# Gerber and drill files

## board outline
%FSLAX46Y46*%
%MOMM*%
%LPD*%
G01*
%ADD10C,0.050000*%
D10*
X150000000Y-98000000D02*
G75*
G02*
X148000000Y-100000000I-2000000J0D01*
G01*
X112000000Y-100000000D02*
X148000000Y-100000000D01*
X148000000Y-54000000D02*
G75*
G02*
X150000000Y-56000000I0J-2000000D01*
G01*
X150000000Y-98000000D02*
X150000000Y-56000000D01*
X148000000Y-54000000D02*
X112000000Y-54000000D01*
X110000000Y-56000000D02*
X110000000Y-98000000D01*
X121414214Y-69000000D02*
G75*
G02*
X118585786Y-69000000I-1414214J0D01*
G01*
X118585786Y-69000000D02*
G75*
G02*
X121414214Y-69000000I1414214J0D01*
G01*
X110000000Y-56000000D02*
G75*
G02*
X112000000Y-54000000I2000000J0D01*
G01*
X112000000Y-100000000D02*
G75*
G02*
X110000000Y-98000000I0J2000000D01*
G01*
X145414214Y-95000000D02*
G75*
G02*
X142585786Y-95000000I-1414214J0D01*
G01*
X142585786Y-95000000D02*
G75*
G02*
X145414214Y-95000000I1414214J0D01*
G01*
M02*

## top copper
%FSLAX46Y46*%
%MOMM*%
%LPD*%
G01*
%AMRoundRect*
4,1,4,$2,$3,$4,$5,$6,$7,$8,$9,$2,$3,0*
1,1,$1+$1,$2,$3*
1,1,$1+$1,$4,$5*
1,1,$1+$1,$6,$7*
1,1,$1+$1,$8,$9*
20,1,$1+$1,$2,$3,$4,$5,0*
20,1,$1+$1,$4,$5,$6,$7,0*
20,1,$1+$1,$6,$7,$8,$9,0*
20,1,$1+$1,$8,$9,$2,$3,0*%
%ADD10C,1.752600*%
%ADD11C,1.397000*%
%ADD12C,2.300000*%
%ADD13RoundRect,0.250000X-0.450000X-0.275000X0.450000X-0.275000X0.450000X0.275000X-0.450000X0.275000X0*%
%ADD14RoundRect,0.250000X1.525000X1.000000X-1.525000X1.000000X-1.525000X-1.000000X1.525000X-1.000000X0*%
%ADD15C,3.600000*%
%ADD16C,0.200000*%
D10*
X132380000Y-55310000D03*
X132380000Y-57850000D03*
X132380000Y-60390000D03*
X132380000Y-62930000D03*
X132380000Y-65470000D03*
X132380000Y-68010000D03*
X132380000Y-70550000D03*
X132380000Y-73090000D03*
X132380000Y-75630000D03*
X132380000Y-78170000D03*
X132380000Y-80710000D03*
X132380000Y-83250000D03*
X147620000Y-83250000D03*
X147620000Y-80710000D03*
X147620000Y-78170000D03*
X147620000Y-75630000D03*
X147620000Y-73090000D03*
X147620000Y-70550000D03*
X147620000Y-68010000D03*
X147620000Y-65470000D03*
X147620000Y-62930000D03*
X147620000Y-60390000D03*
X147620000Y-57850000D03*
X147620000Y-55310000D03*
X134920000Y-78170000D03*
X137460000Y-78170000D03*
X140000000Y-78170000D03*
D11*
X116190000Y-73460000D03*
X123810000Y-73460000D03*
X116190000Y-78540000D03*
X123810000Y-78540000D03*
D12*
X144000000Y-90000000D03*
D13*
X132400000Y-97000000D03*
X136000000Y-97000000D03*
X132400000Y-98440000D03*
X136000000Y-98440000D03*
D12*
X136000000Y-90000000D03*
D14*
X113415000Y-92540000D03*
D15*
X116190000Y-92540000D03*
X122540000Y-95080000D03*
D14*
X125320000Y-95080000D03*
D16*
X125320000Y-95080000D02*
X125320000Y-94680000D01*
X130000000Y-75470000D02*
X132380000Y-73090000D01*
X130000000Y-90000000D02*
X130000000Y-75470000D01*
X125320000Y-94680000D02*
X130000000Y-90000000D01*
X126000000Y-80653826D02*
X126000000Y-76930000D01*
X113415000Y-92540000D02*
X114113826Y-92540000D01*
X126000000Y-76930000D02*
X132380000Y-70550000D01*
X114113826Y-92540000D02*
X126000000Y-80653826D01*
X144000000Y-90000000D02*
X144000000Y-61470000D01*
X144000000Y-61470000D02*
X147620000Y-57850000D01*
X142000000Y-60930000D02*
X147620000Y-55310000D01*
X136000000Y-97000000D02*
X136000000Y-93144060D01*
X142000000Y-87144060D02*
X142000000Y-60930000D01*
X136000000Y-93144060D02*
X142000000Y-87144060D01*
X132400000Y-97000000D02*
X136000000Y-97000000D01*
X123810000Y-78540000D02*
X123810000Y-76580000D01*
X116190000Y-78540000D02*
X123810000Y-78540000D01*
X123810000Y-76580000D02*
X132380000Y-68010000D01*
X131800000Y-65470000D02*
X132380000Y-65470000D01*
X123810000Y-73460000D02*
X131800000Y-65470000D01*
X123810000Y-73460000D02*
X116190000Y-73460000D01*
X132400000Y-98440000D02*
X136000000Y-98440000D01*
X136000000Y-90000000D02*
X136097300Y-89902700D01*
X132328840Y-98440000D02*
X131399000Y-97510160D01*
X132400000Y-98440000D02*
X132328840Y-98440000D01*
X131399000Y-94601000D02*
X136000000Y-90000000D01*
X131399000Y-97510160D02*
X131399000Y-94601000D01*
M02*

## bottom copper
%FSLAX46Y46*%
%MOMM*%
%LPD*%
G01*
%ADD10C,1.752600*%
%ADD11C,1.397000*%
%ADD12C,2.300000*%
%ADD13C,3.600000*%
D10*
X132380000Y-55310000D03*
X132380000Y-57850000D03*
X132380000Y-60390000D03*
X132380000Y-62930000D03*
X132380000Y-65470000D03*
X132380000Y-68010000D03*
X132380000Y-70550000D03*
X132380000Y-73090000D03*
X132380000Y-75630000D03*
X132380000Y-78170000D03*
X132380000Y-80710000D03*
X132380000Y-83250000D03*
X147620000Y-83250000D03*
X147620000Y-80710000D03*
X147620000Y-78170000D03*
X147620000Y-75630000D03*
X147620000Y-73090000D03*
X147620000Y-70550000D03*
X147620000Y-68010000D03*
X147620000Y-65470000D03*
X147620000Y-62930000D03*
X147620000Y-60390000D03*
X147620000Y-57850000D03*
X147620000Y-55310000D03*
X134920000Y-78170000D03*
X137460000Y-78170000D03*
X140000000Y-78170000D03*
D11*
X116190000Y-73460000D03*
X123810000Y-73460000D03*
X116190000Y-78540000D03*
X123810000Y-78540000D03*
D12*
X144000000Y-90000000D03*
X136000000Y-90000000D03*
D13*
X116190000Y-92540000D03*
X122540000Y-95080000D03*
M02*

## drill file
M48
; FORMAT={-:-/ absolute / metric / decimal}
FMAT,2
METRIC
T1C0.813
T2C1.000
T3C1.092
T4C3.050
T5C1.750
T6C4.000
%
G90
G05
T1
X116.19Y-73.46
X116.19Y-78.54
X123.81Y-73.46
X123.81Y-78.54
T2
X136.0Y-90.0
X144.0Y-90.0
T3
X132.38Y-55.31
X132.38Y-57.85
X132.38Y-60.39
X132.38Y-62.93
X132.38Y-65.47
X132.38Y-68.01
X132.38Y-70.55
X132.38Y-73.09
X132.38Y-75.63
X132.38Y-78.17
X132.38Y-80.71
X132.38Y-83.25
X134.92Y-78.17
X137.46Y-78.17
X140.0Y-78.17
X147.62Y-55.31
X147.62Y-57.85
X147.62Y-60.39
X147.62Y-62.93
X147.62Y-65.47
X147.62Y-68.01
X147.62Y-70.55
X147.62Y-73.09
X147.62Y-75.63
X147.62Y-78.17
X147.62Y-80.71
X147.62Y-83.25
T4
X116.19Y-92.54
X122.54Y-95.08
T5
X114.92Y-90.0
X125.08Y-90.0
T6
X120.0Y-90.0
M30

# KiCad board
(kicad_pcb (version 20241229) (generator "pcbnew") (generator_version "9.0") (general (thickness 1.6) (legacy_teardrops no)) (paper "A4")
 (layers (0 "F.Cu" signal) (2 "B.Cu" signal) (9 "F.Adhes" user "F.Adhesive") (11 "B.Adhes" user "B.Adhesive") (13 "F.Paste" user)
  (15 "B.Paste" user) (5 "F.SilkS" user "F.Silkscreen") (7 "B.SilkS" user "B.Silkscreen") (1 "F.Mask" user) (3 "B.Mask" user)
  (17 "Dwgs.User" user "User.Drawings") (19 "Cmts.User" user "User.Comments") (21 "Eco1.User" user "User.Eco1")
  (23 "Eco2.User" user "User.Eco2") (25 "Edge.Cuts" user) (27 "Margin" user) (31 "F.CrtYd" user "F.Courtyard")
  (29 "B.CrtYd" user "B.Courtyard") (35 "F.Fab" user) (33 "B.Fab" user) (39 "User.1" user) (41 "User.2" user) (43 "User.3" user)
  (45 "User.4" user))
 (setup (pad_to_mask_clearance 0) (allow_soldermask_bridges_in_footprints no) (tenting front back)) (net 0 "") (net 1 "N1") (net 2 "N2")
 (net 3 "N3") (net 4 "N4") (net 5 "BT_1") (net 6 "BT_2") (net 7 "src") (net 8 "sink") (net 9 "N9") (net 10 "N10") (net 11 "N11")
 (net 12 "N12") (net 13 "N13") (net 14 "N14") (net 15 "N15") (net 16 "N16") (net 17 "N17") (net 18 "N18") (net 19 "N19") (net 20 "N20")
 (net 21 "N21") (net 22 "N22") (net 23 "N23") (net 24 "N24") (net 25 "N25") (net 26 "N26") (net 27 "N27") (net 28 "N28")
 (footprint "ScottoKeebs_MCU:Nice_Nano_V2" (layer "F.Cu") (at 140 69)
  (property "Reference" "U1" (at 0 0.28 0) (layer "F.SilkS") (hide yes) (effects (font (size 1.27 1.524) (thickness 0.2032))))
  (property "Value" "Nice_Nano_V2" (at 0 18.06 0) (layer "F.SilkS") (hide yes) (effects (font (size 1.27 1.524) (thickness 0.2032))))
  (pad "1" thru_hole circle (at -7.62 -13.69 270) (size 1.7526 1.7526) (drill 1.0922) (layers "*.Cu" "*.Mask") (remove_unused_layers no)
   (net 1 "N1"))
  (pad "2" thru_hole circle (at -7.62 -11.15 270) (size 1.7526 1.7526) (drill 1.0922) (layers "*.Cu" "*.Mask") (remove_unused_layers no)
   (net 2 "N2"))
  (pad "3" thru_hole circle (at -7.62 -8.61 270) (size 1.7526 1.7526) (drill 1.0922) (layers "*.Cu" "*.Mask") (remove_unused_layers no)
   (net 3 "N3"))
  (pad "4" thru_hole circle (at -7.62 -6.07 270) (size 1.7526 1.7526) (drill 1.0922) (layers "*.Cu" "*.Mask") (remove_unused_layers no)
   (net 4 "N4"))
  (pad "5" thru_hole circle (at -7.62 -3.53 270) (size 1.7526 1.7526) (drill 1.0922) (layers "*.Cu" "*.Mask") (remove_unused_layers no)
   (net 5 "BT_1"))
  (pad "6" thru_hole circle (at -7.62 -0.99 270) (size 1.7526 1.7526) (drill 1.0922) (layers "*.Cu" "*.Mask") (remove_unused_layers no)
   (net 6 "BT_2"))
  (pad "7" thru_hole circle (at -7.62 1.55 270) (size 1.7526 1.7526) (drill 1.0922) (layers "*.Cu" "*.Mask") (remove_unused_layers no)
   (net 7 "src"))
  (pad "8" thru_hole circle (at -7.62 4.09 270) (size 1.7526 1.7526) (drill 1.0922) (layers "*.Cu" "*.Mask") (remove_unused_layers no)
   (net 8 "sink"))
  (pad "9" thru_hole circle (at -7.62 6.63 270) (size 1.7526 1.7526) (drill 1.0922) (layers "*.Cu" "*.Mask") (remove_unused_layers no)
   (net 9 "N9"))
  (pad "10" thru_hole circle (at -7.62 9.17 270) (size 1.7526 1.7526) (drill 1.0922) (layers "*.Cu" "*.Mask") (remove_unused_layers no)
   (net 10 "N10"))
  (pad "11" thru_hole circle (at -7.62 11.71 270) (size 1.7526 1.7526) (drill 1.0922) (layers "*.Cu" "*.Mask") (remove_unused_layers no)
   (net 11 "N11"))
  (pad "12" thru_hole circle (at -7.62 14.25 270) (size 1.7526 1.7526) (drill 1.0922) (layers "*.Cu" "*.Mask") (remove_unused_layers no)
   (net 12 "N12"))
  (pad "13" thru_hole circle (at 7.62 14.25 270) (size 1.7526 1.7526) (drill 1.0922) (layers "*.Cu" "*.Mask") (remove_unused_layers no)
   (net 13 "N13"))
  (pad "14" thru_hole circle (at 7.62 11.71 270) (size 1.7526 1.7526) (drill 1.0922) (layers "*.Cu" "*.Mask") (remove_unused_layers no)
   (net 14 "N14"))
  (pad "15" thru_hole circle (at 7.62 9.17 270) (size 1.7526 1.7526) (drill 1.0922) (layers "*.Cu" "*.Mask") (remove_unused_layers no)
   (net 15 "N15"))
  (pad "16" thru_hole circle (at 7.62 6.63 270) (size 1.7526 1.7526) (drill 1.0922) (layers "*.Cu" "*.Mask") (remove_unused_layers no)
   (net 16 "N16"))
  (pad "17" thru_hole circle (at 7.62 4.09 270) (size 1.7526 1.7526) (drill 1.0922) (layers "*.Cu" "*.Mask") (remove_unused_layers no)
   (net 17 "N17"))
  (pad "18" thru_hole circle (at 7.62 1.55 270) (size 1.7526 1.7526) (drill 1.0922) (layers "*.Cu" "*.Mask") (remove_unused_layers no)
   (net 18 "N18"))
  (pad "19" thru_hole circle (at 7.62 -0.99 270) (size 1.7526 1.7526) (drill 1.0922) (layers "*.Cu" "*.Mask") (remove_unused_layers no)
   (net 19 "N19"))
  (pad "20" thru_hole circle (at 7.62 -3.53 270) (size 1.7526 1.7526) (drill 1.0922) (layers "*.Cu" "*.Mask") (remove_unused_layers no)
   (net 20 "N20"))
  (pad "21" thru_hole circle (at 7.62 -6.07 270) (size 1.7526 1.7526) (drill 1.0922) (layers "*.Cu" "*.Mask") (remove_unused_layers no)
   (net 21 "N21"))
  (pad "22" thru_hole circle (at 7.62 -8.61 270) (size 1.7526 1.7526) (drill 1.0922) (layers "*.Cu" "*.Mask") (remove_unused_layers no)
   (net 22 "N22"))
  (pad "23" thru_hole circle (at 7.62 -11.15 270) (size 1.7526 1.7526) (drill 1.0922) (layers "*.Cu" "*.Mask") (remove_unused_layers no)
   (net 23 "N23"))
  (pad "24" thru_hole circle (at 7.62 -13.69 270) (size 1.7526 1.7526) (drill 1.0922) (layers "*.Cu" "*.Mask") (remove_unused_layers no)
   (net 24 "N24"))
  (pad "25" thru_hole circle (at -5.08 9.17) (size 1.7526 1.7526) (drill 1.0922) (layers "*.Cu" "*.Mask") (remove_unused_layers no)
   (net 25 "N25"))
  (pad "26" thru_hole circle (at -2.54 9.17) (size 1.7526 1.7526) (drill 1.0922) (layers "*.Cu" "*.Mask") (remove_unused_layers no)
   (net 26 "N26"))
  (pad "27" thru_hole circle (at 0 9.17) (size 1.7526 1.7526) (drill 1.0922) (layers "*.Cu" "*.Mask") (remove_unused_layers no)
   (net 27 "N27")))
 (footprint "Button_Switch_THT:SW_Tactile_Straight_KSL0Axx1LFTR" (layer "F.Cu") (at 116.19 73.46)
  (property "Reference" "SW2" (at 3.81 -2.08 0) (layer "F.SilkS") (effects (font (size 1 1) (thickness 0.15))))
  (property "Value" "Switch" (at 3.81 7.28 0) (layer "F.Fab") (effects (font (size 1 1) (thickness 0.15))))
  (pad "1" thru_hole circle (at 0 0) (size 1.397 1.397) (drill 0.8128) (layers "*.Cu" "*.Mask") (remove_unused_layers no) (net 5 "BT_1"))
  (pad "1" thru_hole circle (at 7.62 0) (size 1.397 1.397) (drill 0.8128) (layers "*.Cu" "*.Mask") (remove_unused_layers no) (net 5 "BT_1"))
  (pad "2" thru_hole circle (at 0 5.08) (size 1.397 1.397) (drill 0.8128) (layers "*.Cu" "*.Mask") (remove_unused_layers no) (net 6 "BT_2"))
  (pad "2" thru_hole circle (at 7.62 5.08) (size 1.397 1.397) (drill 0.8128) (layers "*.Cu" "*.Mask") (remove_unused_layers no)
   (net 6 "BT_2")))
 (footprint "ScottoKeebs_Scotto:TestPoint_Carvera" (layer "F.Cu") (at 144 90)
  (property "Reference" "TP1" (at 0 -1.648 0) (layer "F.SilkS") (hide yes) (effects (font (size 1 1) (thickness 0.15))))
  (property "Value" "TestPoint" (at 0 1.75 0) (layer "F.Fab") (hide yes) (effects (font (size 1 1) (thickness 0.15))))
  (pad "1" thru_hole circle (at 0 0) (size 2.3 2.3) (drill 1) (layers "*.Cu" "*.Mask") (remove_unused_layers no) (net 23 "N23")))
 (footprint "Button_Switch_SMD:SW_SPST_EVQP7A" (layer "F.Cu") (at 134.2 97.72)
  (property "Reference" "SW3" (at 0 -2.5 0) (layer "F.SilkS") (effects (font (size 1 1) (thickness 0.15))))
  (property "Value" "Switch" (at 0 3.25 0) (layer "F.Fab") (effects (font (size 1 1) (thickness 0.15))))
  (pad "1" smd roundrect (at -1.8 -0.72) (size 1.4 1.05) (layers "F.Cu" "F.Mask" "F.Paste") (roundrect_rratio 0.2380952381) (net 24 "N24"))
  (pad "1" smd roundrect (at 1.8 -0.72) (size 1.4 1.05) (layers "F.Cu" "F.Mask" "F.Paste") (roundrect_rratio 0.2380952381) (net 24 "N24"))
  (pad "2" smd roundrect (at -1.8 0.72) (size 1.4 1.05) (layers "F.Cu" "F.Mask" "F.Paste") (roundrect_rratio 0.2380952381) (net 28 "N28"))
  (pad "2" smd roundrect (at 1.8 0.72) (size 1.4 1.05) (layers "F.Cu" "F.Mask" "F.Paste") (roundrect_rratio 0.2380952381) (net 28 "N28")))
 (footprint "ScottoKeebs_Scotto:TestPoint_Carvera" (layer "F.Cu") (at 136 90)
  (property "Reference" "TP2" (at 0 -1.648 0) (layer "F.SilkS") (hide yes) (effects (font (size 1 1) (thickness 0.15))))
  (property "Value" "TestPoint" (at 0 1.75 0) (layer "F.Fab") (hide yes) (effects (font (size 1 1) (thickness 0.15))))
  (pad "1" thru_hole circle (at 0 0) (size 2.3 2.3) (drill 1) (layers "*.Cu" "*.Mask") (remove_unused_layers no) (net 28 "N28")))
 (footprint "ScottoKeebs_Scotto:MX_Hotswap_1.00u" (layer "F.Cu") (at 119.365 93.81)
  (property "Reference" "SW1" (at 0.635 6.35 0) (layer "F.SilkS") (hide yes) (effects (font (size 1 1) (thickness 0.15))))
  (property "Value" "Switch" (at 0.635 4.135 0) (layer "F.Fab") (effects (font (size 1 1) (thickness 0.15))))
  (pad "" smd roundrect (at -6.45 -1.27 180) (size 2.55 2.5) (layers "F.Mask" "F.Paste") (roundrect_rratio 0.1))
  (pad "" np_thru_hole circle (at -4.445 -3.81 180) (size 1.75 1.75) (drill 1.75) (layers "*.Cu" "*.Mask") (clearance 0.1))
  (pad "" np_thru_hole circle (at 0.635 -3.81 180) (size 4 4) (drill 4) (layers "*.Cu" "*.Mask"))
  (pad "" np_thru_hole circle (at 5.715 -3.81 180) (size 1.75 1.75) (drill 1.75) (layers "*.Cu" "*.Mask"))
  (pad "" smd roundrect (at 6.477 1.27 180) (size 2.55 2.5) (layers "F.Mask" "F.Paste") (roundrect_rratio 0.1))
  (pad "1" smd roundrect (at -5.95 -1.27 180) (size 3.55 2.5) (layers "F.Cu") (roundrect_rratio 0.1) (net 7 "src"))
  (pad "1" thru_hole circle (at -3.175 -1.27 180) (size 3.6 3.6) (drill 3.05) (layers "*.Cu" "*.Mask") (remove_unused_layers no)
   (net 7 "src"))
  (pad "2" thru_hole circle (at 3.175 1.27 180) (size 3.6 3.6) (drill 3.05) (layers "*.Cu" "*.Mask") (remove_unused_layers no)
   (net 8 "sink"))
  (pad "2" smd roundrect (at 5.955 1.27 180) (size 3.55 2.5) (layers "F.Cu") (roundrect_rratio 0.1) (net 8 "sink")))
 (gr_arc (start 150 98) (mid 149.414214 99.414214) (end 148 100) (stroke (width 0.05) (type default)) (layer "Edge.Cuts"))
 (gr_line (start 112 100) (end 148 100) (stroke (width 0.05) (type default)) (layer "Edge.Cuts"))
 (gr_arc (start 148 54) (mid 149.414214 54.585786) (end 150 56) (stroke (width 0.05) (type default)) (layer "Edge.Cuts"))
 (gr_line (start 150 98) (end 150 56) (stroke (width 0.05) (type default)) (layer "Edge.Cuts"))
 (gr_line (start 148 54) (end 112 54) (stroke (width 0.05) (type default)) (layer "Edge.Cuts"))
 (gr_line (start 110 56) (end 110 98) (stroke (width 0.05) (type default)) (layer "Edge.Cuts"))
 (gr_circle (center 120 69) (end 121 68) (stroke (width 0.05) (type default)) (fill no) (layer "Edge.Cuts"))
 (gr_arc (start 110 56) (mid 110.585786 54.585786) (end 112 54) (stroke (width 0.05) (type default)) (layer "Edge.Cuts"))
 (gr_arc (start 112 100) (mid 110.585786 99.414214) (end 110 98) (stroke (width 0.05) (type default)) (layer "Edge.Cuts"))
 (gr_circle (center 144 95) (end 145 94) (stroke (width 0.05) (type default)) (fill no) (layer "Edge.Cuts"))
 (segment (start 125.32 95.08) (end 125.32 94.68) (width 0.2) (layer "F.Cu") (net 8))
 (segment (start 130 75.47) (end 132.38 73.09) (width 0.2) (layer "F.Cu") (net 8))
 (segment (start 130 90) (end 130 75.47) (width 0.2) (layer "F.Cu") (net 8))
 (segment (start 125.32 94.68) (end 130 90) (width 0.2) (layer "F.Cu") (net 8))
 (segment (start 126 80.653826) (end 126 76.93) (width 0.2) (layer "F.Cu") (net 7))
 (segment (start 113.415 92.54) (end 114.113826 92.54) (width 0.2) (layer "F.Cu") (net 7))
 (segment (start 126 76.93) (end 132.38 70.55) (width 0.2) (layer "F.Cu") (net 7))
 (segment (start 114.113826 92.54) (end 126 80.653826) (width 0.2) (layer "F.Cu") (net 7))
 (segment (start 144 90) (end 144 61.47) (width 0.2) (layer "F.Cu") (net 23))
 (segment (start 144 61.47) (end 147.62 57.85) (width 0.2) (layer "F.Cu") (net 23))
 (segment (start 142 60.93) (end 147.62 55.31) (width 0.2) (layer "F.Cu") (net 24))
 (segment (start 136 97) (end 136 93.14406) (width 0.2) (layer "F.Cu") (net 24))
 (segment (start 142 87.14406) (end 142 60.93) (width 0.2) (layer "F.Cu") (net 24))
 (segment (start 136 93.14406) (end 142 87.14406) (width 0.2) (layer "F.Cu") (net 24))
 (segment (start 132.4 97) (end 136 97) (width 0.2) (layer "F.Cu") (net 24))
 (segment (start 123.81 78.54) (end 123.81 76.58) (width 0.2) (layer "F.Cu") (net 6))
 (segment (start 116.19 78.54) (end 123.81 78.54) (width 0.2) (layer "F.Cu") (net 6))
 (segment (start 123.81 76.58) (end 132.38 68.01) (width 0.2) (layer "F.Cu") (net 6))
 (segment (start 131.8 65.47) (end 132.38 65.47) (width 0.2) (layer "F.Cu") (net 5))
 (segment (start 123.81 73.46) (end 131.8 65.47) (width 0.2) (layer "F.Cu") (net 5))
 (segment (start 123.81 73.46) (end 116.19 73.46) (width 0.2) (layer "F.Cu") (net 5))
 (segment (start 132.4 98.44) (end 136 98.44) (width 0.2) (layer "F.Cu") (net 28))
 (segment (start 136 90) (end 136.0973 89.9027) (width 0.2) (layer "F.Cu") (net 28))
 (segment (start 132.32884 98.44) (end 131.399 97.51016) (width 0.2) (layer "F.Cu") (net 28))
 (segment (start 132.4 98.44) (end 132.32884 98.44) (width 0.2) (layer "F.Cu") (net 28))
 (segment (start 131.399 94.601) (end 136 90) (width 0.2) (layer "F.Cu") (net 28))
 (segment (start 131.399 97.51016) (end 131.399 94.601) (width 0.2) (layer "F.Cu") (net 28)))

